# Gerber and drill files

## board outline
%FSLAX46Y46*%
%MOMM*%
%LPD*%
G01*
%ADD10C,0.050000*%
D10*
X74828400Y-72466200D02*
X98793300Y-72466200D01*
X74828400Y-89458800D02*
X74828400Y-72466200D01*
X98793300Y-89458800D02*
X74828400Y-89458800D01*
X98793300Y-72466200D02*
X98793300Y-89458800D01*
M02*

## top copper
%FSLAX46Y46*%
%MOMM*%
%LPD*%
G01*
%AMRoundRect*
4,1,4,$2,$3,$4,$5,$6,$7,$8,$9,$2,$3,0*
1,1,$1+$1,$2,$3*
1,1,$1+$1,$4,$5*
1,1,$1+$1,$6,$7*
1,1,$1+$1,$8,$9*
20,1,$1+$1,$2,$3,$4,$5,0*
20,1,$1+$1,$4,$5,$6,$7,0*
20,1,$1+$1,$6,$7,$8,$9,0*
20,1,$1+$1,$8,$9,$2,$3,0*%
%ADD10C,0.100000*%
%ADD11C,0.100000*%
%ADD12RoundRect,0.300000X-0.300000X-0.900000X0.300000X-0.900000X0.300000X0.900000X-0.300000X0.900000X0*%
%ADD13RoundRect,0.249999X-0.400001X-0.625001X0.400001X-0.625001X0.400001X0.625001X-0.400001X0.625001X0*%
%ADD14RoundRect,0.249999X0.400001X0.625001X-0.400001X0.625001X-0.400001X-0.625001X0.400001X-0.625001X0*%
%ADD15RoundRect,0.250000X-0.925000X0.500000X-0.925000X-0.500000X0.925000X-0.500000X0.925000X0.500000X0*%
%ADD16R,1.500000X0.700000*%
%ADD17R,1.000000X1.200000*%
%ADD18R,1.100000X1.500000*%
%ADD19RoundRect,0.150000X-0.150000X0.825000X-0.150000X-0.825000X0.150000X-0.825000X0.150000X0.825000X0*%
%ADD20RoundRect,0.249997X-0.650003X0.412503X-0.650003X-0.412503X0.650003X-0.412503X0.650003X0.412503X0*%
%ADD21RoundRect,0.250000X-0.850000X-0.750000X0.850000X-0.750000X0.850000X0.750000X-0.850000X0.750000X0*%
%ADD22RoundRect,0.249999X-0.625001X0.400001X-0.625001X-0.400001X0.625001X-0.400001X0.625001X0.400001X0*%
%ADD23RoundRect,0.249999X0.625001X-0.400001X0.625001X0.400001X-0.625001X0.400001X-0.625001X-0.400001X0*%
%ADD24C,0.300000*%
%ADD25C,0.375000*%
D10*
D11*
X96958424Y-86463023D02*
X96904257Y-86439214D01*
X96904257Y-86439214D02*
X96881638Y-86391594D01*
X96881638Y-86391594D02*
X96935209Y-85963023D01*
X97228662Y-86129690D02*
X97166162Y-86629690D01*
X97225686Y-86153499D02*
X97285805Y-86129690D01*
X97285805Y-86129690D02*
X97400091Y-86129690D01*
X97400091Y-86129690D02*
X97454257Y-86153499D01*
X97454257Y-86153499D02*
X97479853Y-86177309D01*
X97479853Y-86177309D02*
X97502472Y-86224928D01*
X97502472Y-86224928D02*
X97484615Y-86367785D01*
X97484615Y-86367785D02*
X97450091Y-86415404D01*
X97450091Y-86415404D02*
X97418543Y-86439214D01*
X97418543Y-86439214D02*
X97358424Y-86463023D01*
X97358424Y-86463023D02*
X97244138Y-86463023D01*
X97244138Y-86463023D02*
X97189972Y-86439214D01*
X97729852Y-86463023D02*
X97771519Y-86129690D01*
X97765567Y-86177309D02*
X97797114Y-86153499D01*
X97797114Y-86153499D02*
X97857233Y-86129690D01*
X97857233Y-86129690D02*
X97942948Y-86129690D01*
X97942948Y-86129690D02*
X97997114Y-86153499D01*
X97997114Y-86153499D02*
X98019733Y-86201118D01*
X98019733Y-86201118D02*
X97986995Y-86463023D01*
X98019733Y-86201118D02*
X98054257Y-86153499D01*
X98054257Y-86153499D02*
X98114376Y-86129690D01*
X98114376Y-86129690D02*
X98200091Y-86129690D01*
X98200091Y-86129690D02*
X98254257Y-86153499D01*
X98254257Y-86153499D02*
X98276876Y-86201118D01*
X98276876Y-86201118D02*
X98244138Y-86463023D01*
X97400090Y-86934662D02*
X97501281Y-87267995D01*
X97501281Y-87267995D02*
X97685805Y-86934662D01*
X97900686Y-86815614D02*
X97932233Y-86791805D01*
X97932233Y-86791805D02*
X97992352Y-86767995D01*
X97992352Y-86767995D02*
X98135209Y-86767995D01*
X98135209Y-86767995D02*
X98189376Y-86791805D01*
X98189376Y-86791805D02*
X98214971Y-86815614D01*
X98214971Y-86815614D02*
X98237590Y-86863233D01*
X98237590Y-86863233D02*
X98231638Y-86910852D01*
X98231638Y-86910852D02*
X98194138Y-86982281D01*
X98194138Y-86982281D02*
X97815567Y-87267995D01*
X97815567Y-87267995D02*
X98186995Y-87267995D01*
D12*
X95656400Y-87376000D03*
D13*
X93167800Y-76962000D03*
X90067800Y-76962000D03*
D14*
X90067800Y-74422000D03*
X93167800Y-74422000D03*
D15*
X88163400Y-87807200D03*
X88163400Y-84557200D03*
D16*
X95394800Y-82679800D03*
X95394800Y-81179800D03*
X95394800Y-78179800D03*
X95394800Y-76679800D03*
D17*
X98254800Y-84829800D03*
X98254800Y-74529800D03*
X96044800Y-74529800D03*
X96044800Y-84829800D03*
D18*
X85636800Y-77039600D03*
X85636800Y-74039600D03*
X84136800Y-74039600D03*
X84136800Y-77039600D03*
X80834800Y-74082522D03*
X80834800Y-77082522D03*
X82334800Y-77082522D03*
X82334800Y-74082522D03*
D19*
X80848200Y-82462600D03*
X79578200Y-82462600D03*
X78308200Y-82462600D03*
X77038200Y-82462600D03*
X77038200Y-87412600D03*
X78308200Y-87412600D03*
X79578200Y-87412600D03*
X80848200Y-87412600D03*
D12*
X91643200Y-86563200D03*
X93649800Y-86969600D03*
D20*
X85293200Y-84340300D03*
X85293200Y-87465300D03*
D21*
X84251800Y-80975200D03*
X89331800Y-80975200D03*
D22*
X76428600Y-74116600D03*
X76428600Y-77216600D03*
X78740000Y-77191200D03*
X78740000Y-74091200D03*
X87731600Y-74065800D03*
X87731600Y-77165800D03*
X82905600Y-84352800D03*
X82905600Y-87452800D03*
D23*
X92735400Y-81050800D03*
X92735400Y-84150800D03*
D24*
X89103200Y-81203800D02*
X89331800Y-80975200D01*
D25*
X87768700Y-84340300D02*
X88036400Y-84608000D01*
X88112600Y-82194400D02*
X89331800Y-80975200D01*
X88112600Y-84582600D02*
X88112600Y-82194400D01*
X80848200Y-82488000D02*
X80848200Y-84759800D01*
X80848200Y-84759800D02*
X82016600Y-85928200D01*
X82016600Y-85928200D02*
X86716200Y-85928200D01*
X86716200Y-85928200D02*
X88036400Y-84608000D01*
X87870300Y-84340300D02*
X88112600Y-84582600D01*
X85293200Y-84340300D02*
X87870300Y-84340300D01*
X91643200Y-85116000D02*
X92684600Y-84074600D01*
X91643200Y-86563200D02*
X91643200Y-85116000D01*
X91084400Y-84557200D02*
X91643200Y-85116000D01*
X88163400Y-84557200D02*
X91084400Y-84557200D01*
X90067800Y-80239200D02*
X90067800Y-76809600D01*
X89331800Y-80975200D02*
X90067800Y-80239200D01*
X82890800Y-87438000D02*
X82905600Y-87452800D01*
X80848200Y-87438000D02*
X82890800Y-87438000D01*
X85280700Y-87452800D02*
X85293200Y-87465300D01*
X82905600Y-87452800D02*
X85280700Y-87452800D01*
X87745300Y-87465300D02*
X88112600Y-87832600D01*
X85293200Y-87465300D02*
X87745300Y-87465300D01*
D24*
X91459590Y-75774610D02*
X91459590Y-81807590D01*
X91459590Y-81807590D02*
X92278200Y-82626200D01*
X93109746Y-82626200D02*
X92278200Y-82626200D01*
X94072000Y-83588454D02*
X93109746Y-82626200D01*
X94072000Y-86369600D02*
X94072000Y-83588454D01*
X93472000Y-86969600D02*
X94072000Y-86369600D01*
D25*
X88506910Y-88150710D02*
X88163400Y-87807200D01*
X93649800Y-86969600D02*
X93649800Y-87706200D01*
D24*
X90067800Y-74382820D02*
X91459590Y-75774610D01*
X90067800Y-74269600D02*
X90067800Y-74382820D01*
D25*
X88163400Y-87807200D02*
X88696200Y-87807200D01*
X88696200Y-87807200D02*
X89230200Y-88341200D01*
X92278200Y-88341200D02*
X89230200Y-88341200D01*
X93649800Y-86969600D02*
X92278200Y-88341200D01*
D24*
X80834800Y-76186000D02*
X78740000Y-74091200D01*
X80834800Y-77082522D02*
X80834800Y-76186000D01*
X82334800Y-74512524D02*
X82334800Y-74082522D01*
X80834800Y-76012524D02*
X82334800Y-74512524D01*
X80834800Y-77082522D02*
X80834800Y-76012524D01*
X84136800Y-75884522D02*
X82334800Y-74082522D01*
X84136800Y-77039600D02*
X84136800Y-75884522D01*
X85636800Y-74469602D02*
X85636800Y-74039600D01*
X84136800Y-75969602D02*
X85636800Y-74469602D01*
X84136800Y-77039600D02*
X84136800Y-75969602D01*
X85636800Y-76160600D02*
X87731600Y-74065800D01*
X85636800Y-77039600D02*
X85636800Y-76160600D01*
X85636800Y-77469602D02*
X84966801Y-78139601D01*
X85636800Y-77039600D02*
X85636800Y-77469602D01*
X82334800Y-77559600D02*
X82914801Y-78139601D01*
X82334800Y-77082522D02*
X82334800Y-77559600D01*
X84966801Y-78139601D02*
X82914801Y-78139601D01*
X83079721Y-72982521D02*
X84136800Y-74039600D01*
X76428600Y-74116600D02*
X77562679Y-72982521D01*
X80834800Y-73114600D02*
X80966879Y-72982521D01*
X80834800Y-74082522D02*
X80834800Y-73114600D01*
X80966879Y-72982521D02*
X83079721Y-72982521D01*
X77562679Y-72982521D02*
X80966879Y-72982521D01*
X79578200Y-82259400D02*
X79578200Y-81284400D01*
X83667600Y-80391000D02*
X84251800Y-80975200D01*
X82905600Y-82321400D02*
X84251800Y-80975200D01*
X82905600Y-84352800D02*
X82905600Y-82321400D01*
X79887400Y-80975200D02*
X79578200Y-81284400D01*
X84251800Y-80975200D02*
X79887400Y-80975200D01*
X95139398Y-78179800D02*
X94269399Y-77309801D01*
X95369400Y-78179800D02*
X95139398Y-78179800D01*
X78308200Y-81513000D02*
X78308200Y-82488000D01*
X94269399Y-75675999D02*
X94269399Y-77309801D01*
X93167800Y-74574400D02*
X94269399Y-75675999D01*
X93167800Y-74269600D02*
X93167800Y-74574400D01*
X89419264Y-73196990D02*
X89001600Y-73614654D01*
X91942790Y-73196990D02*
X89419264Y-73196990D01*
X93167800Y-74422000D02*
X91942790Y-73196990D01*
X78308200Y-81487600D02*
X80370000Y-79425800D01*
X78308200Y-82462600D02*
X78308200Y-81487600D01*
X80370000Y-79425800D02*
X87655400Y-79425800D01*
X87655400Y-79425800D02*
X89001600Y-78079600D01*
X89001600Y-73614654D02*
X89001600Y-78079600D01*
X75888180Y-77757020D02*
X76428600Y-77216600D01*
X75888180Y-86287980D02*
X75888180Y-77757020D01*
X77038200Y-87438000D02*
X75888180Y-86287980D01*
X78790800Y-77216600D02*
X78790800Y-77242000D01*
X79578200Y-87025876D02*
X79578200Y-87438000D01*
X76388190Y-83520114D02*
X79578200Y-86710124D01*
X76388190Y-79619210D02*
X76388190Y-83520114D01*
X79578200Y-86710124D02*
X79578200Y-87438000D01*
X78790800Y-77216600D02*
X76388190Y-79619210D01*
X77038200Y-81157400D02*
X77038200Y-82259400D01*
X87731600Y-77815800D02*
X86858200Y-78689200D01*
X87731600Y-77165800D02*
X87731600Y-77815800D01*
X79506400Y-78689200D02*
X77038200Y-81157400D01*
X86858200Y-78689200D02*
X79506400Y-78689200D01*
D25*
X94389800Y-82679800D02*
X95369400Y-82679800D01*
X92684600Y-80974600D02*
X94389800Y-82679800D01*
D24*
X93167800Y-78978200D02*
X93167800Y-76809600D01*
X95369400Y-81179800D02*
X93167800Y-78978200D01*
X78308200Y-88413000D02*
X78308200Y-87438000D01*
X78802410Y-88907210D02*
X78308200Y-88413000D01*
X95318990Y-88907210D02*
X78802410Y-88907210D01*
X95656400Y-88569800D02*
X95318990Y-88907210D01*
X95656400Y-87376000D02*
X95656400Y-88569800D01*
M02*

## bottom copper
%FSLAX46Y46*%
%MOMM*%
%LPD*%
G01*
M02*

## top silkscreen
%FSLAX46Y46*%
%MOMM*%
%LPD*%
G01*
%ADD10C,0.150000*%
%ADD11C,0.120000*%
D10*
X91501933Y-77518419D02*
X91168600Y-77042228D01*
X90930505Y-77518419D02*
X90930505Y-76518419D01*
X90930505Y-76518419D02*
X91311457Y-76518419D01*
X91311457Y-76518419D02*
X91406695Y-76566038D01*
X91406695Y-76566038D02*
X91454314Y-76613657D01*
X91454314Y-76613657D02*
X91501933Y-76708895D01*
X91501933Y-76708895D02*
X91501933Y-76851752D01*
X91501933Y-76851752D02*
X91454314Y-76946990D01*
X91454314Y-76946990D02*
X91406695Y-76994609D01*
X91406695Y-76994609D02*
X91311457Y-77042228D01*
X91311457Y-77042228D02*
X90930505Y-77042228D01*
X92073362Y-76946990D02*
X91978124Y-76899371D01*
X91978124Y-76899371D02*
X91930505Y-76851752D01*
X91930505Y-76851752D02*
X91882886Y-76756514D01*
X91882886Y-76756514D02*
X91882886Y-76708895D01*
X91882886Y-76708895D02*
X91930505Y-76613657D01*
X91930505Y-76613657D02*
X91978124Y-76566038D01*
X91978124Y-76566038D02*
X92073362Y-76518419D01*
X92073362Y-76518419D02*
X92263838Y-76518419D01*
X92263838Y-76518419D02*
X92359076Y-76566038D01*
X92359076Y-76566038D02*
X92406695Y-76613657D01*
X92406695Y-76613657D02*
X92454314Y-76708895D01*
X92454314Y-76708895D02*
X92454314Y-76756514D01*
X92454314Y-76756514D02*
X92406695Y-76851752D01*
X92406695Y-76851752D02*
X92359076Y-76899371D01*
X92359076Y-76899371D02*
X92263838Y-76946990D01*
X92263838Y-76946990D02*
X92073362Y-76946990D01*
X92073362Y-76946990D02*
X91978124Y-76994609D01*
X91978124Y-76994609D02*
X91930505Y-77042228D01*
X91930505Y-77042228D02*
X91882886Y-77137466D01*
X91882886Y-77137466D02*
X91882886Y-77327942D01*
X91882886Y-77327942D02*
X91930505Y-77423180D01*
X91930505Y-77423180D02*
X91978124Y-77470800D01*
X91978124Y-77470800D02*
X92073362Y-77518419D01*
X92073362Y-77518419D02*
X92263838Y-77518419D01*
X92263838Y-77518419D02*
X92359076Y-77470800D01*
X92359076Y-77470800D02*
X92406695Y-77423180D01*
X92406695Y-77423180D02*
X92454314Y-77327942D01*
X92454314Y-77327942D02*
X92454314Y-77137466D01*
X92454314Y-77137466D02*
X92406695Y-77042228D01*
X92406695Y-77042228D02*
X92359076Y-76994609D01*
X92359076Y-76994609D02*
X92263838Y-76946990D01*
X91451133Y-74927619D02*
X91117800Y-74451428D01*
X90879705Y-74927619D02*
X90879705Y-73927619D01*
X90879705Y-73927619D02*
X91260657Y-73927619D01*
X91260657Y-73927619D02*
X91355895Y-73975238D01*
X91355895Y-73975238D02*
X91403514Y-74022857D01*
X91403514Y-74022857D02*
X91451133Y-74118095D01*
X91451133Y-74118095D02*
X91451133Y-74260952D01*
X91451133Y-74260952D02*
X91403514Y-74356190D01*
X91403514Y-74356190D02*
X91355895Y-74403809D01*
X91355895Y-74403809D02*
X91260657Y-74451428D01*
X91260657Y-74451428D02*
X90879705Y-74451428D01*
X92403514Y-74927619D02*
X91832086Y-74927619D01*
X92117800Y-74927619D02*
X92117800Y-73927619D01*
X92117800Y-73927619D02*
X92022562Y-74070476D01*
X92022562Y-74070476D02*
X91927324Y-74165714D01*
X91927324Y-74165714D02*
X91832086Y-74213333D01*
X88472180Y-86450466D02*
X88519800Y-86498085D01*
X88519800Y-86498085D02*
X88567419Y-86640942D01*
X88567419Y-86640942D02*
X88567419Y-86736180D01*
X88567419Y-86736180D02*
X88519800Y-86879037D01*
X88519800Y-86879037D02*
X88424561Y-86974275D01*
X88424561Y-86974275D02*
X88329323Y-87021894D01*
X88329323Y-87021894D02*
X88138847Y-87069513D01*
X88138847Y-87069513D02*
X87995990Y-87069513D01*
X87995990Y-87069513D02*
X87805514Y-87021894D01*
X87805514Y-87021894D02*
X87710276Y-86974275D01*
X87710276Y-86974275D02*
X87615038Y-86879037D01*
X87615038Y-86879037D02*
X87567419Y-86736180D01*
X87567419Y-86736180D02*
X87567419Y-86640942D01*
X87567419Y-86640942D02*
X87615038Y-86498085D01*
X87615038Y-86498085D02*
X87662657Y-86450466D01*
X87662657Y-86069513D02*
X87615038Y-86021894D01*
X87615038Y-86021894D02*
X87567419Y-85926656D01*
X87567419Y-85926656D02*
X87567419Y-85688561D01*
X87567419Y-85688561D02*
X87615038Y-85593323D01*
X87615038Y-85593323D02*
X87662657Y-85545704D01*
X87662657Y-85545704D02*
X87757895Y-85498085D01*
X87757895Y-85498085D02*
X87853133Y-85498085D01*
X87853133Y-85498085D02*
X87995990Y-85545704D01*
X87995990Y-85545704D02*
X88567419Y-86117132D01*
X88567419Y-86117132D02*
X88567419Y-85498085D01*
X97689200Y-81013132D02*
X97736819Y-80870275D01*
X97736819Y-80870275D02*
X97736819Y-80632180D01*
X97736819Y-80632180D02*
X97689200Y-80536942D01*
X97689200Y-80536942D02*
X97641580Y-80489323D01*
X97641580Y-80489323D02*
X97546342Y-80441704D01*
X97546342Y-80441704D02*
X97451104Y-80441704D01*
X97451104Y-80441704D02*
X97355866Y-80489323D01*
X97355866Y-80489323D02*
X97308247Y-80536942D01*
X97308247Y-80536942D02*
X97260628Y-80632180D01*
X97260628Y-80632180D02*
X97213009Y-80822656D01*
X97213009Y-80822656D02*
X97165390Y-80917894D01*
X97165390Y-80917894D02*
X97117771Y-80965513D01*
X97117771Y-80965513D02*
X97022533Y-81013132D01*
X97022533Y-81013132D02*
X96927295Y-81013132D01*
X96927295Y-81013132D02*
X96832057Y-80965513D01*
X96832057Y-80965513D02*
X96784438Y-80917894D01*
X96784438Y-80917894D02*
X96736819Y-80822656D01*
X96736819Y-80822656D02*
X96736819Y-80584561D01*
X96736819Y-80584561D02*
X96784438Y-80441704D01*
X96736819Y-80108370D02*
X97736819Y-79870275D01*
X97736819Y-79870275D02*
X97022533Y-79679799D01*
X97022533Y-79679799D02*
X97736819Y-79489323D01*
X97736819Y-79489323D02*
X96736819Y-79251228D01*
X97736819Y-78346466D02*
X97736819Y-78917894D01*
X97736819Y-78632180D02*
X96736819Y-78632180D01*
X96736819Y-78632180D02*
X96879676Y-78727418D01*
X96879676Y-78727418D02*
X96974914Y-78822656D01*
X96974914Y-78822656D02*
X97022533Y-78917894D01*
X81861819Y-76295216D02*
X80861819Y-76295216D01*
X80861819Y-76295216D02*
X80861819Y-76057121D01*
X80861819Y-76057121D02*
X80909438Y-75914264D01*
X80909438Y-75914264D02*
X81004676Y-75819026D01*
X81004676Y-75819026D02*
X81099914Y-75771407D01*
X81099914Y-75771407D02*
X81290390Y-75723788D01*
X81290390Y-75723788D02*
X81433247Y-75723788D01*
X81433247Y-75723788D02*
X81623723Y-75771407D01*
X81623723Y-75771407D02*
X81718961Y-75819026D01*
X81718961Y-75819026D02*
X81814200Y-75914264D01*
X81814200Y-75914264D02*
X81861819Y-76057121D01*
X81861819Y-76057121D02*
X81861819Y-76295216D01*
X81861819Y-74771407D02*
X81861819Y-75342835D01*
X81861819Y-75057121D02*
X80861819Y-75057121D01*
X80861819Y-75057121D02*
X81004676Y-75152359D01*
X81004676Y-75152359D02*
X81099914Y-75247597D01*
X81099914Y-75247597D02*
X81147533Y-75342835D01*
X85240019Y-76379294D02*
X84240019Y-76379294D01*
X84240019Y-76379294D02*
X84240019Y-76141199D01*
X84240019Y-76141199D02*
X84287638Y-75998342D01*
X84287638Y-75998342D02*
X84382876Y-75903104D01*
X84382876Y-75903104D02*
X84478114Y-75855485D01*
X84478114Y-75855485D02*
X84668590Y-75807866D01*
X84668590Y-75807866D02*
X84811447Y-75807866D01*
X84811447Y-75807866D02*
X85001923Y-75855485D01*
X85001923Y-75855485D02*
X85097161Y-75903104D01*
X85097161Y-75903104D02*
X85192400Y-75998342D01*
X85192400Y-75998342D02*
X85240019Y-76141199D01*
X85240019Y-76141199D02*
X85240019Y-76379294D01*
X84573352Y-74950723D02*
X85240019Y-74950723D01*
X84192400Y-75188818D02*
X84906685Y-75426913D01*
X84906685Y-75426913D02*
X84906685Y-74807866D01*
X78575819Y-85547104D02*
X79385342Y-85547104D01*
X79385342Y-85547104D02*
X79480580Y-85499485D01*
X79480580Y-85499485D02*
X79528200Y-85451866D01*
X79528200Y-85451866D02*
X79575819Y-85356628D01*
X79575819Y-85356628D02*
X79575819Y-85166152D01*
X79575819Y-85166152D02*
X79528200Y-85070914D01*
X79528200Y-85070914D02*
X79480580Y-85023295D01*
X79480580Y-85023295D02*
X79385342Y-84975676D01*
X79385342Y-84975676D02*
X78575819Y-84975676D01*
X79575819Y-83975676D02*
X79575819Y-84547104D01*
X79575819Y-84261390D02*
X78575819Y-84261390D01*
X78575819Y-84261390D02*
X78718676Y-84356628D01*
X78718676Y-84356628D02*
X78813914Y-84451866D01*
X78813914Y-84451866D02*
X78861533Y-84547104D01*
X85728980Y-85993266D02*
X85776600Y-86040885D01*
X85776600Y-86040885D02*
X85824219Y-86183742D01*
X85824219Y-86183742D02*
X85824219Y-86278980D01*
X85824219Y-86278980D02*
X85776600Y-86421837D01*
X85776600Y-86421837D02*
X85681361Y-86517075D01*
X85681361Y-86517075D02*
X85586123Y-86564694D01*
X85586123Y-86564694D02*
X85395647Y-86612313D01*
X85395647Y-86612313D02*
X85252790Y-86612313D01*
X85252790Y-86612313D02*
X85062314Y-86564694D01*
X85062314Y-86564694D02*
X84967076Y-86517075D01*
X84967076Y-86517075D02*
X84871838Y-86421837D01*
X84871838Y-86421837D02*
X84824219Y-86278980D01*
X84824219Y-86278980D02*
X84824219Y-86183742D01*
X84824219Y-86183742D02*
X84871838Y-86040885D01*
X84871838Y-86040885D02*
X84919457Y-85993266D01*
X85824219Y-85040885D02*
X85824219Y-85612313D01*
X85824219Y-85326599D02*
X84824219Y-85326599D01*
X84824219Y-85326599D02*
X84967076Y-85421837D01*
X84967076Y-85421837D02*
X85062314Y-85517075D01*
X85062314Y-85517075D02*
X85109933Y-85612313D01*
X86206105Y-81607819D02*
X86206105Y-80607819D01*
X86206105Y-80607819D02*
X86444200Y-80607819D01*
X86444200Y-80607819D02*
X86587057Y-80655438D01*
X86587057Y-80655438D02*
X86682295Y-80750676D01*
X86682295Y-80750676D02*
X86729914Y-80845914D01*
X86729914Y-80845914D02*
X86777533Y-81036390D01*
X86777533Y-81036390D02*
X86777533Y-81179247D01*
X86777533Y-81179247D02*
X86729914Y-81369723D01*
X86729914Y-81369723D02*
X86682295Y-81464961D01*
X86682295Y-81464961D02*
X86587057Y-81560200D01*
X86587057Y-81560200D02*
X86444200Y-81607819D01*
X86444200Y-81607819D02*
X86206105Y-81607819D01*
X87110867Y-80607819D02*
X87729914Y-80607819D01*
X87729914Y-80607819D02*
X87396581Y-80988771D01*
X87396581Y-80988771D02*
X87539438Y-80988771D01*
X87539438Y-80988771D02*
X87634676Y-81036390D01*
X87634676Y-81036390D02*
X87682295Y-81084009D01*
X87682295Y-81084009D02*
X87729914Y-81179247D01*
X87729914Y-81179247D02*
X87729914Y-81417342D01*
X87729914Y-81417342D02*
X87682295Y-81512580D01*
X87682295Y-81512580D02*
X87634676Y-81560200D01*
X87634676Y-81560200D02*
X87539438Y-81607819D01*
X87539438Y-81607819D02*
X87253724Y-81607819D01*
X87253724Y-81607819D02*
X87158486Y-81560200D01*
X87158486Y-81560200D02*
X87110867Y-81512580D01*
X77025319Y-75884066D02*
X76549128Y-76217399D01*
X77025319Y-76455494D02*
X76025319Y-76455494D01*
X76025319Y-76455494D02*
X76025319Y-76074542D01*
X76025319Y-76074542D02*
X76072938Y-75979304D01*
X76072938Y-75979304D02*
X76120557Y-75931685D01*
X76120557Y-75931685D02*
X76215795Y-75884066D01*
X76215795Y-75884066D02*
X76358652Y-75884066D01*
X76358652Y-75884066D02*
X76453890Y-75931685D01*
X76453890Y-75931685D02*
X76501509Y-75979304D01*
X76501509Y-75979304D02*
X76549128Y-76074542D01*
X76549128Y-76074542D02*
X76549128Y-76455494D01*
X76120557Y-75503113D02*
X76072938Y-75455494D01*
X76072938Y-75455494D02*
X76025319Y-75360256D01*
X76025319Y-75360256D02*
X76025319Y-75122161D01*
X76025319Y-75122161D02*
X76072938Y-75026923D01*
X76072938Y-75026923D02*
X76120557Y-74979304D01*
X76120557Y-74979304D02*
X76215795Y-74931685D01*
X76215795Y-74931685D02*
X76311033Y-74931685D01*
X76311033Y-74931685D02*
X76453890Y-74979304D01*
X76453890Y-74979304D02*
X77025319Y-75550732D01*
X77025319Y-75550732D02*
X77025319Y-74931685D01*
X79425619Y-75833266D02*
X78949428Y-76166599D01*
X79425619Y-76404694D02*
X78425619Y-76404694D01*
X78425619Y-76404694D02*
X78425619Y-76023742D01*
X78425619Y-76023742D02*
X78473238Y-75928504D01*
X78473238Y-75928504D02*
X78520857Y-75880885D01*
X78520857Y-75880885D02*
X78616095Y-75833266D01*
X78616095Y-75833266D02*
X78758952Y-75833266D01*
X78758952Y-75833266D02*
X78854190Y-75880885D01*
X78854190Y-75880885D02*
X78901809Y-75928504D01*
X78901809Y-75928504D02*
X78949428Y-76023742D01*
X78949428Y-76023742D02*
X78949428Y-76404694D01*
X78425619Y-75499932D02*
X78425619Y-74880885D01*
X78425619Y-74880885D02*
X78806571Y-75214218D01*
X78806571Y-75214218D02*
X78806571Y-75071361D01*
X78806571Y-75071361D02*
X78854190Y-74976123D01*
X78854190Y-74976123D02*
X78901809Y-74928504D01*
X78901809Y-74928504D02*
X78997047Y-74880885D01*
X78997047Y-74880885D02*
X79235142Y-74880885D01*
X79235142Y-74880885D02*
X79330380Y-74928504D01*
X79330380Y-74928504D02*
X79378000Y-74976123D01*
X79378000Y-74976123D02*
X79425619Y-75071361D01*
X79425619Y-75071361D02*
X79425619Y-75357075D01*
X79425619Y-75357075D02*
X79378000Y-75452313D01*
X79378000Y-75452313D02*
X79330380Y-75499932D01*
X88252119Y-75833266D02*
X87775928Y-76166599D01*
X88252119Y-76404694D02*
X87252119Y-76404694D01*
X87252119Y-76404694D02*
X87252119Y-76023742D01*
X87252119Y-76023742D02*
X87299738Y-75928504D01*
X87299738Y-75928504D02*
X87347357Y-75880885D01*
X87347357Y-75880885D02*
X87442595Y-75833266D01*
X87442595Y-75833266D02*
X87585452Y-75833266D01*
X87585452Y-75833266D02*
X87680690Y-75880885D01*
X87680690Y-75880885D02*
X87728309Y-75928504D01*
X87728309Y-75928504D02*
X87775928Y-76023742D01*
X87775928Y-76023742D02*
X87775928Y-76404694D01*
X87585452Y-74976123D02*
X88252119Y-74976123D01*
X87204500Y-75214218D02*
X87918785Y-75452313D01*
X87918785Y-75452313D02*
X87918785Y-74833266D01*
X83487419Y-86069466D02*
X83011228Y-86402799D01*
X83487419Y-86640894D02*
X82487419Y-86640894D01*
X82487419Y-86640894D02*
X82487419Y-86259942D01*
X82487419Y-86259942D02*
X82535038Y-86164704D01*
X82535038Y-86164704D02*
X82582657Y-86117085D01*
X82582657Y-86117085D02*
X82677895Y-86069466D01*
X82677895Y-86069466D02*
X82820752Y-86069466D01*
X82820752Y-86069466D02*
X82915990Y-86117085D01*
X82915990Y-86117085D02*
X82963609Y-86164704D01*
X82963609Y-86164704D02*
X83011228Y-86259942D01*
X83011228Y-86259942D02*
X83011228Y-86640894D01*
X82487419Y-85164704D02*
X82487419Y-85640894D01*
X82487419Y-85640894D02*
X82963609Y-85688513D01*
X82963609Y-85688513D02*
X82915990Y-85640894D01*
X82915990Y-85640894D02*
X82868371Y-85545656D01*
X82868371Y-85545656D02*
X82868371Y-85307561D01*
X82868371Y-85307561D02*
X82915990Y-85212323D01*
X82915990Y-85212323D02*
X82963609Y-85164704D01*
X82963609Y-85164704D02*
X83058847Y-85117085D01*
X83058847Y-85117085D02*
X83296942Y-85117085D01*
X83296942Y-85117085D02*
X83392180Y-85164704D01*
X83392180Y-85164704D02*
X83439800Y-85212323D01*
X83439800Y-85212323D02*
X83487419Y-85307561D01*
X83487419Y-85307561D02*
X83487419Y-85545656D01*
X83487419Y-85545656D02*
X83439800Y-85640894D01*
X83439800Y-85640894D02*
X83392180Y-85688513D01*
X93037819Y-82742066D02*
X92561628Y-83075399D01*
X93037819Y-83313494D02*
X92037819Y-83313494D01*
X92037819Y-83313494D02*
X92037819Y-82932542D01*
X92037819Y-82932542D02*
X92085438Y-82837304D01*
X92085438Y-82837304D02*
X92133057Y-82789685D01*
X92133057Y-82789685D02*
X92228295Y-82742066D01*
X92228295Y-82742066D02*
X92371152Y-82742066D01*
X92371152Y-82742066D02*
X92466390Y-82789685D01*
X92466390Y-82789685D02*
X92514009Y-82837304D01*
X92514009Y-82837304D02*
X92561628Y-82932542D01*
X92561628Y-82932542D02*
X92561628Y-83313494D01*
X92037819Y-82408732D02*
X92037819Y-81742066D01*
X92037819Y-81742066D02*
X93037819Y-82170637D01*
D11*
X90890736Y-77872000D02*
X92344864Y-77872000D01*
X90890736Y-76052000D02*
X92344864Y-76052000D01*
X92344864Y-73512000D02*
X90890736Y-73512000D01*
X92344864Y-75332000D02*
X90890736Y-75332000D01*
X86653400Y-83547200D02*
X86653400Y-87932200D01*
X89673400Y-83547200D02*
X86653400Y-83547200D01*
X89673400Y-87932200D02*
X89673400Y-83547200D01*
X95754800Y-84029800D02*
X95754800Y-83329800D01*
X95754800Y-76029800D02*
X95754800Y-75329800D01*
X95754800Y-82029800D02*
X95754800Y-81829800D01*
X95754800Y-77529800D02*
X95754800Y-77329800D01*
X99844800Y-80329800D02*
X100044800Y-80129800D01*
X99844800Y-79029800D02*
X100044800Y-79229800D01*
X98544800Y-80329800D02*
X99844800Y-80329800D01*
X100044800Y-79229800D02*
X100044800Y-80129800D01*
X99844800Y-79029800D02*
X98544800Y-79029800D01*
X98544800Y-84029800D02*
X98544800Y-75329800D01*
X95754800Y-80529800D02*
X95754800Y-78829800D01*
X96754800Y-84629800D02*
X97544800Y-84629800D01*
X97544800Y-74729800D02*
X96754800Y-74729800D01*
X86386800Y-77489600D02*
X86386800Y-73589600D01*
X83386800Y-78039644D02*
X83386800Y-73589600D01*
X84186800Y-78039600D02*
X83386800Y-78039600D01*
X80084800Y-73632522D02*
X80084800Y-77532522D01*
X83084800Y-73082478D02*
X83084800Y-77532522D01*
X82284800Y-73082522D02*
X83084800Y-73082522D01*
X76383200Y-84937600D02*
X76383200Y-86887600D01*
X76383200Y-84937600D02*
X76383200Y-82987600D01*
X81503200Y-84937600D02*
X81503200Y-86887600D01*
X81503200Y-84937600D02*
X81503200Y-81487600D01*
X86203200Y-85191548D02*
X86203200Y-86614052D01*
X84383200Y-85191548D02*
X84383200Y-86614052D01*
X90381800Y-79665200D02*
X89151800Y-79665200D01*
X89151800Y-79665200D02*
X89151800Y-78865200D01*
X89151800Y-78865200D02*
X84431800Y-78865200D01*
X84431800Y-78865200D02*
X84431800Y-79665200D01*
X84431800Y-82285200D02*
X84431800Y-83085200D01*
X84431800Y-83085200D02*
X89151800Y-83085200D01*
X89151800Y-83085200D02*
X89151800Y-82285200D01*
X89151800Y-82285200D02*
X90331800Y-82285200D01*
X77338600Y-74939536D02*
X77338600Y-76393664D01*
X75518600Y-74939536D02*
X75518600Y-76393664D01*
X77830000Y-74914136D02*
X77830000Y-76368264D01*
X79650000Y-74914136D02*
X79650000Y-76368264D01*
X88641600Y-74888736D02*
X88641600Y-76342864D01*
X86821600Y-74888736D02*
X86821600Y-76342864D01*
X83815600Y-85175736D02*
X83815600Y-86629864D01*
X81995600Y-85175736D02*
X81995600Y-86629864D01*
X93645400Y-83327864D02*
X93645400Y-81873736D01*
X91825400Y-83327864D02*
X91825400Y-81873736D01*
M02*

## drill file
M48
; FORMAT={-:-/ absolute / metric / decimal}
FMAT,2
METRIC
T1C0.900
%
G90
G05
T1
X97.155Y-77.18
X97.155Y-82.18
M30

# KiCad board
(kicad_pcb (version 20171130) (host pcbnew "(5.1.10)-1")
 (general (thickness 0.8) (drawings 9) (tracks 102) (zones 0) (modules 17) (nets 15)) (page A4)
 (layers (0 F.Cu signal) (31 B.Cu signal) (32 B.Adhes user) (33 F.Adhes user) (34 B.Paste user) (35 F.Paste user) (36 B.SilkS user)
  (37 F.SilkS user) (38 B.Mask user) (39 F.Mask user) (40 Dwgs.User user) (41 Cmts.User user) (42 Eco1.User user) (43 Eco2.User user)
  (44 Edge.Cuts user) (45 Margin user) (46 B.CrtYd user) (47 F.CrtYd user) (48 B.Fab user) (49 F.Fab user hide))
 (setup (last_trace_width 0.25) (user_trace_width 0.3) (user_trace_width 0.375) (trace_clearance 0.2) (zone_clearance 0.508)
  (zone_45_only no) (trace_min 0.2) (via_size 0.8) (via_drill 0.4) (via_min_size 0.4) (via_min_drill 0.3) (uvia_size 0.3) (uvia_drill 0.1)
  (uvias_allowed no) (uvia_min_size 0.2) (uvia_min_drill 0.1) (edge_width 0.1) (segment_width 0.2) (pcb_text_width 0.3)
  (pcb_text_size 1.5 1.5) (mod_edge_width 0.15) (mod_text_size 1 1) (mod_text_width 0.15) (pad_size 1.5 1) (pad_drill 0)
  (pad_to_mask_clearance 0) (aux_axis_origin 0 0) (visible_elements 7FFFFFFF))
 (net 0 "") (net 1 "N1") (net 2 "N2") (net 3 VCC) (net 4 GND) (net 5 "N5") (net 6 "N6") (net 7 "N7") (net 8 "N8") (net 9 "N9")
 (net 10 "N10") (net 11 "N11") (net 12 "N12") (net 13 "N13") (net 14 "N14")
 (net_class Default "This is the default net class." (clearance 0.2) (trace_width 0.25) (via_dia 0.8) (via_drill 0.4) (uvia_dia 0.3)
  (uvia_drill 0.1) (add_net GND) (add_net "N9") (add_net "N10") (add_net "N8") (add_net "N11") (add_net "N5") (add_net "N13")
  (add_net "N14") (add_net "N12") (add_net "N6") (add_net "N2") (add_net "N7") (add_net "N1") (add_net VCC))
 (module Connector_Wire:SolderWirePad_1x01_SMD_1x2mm (layer F.Cu) (at 95.6564 87.376)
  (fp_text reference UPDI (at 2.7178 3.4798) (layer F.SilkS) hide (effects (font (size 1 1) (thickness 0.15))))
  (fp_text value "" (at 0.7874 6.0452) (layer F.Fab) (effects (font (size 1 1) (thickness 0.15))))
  (pad 1 smd roundrect (at 0 0) (size 1.2 2.4) (layers F.Cu F.Mask) (roundrect_rratio 0.25) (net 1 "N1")))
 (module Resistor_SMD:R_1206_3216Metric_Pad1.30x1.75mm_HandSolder (layer F.Cu) (at 91.6178 76.962)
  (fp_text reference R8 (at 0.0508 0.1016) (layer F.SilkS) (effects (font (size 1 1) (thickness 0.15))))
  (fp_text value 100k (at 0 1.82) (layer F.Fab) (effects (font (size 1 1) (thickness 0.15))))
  (fp_line (start -0.727064 0.91) (end 0.727064 0.91) (layer F.SilkS) (width 0.12))
  (fp_line (start -0.727064 -0.91) (end 0.727064 -0.91) (layer F.SilkS) (width 0.12))
  (pad 2 smd roundrect (at 1.55 0) (size 1.3 1.75) (layers F.Cu F.Paste F.Mask) (roundrect_rratio 0.1923069230769231) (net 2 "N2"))
  (pad 1 smd roundrect (at -1.55 0) (size 1.3 1.75) (layers F.Cu F.Paste F.Mask) (roundrect_rratio 0.1923069230769231) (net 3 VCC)))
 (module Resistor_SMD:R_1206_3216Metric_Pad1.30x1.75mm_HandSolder (layer F.Cu) (at 91.6178 74.422 180)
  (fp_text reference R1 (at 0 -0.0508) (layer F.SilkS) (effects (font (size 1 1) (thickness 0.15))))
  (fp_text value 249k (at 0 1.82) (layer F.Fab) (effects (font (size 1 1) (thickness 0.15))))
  (fp_line (start -0.727064 0.91) (end 0.727064 0.91) (layer F.SilkS) (width 0.12))
  (fp_line (start -0.727064 -0.91) (end 0.727064 -0.91) (layer F.SilkS) (width 0.12))
  (pad 2 smd roundrect (at 1.55 0 180) (size 1.3 1.75) (layers F.Cu F.Paste F.Mask) (roundrect_rratio 0.1923069230769231) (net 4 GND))
  (pad 1 smd roundrect (at -1.55 0 180) (size 1.3 1.75) (layers F.Cu F.Paste F.Mask) (roundrect_rratio 0.1923069230769231) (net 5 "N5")))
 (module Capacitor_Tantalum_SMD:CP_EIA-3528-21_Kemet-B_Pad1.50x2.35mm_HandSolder (layer F.Cu) (at 88.1634 86.1822 270)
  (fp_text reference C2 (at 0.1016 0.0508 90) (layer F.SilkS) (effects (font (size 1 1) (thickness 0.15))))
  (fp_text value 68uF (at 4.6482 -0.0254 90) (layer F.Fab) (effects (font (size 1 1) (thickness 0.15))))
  (fp_line (start -2.635 1.51) (end 1.75 1.51) (layer F.SilkS) (width 0.12))
  (fp_line (start -2.635 -1.51) (end -2.635 1.51) (layer F.SilkS) (width 0.12))
  (fp_line (start 1.75 -1.51) (end -2.635 -1.51) (layer F.SilkS) (width 0.12))
  (pad 2 smd roundrect (at 1.625 0 270) (size 1.5 2.35) (layers F.Cu F.Paste F.Mask) (roundrect_rratio 0.1666666666666667) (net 4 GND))
  (pad 1 smd roundrect (at -1.625 0 270) (size 1.5 2.35) (layers F.Cu F.Paste F.Mask) (roundrect_rratio 0.1666666666666667) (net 3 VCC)))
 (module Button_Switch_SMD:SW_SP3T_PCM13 (layer F.Cu) (at 96.8248 79.6798 90)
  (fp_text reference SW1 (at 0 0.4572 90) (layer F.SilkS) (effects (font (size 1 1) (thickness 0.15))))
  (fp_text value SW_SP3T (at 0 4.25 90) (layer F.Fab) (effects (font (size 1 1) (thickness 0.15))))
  (fp_line (start -4.35 -1.07) (end -3.65 -1.07) (layer F.SilkS) (width 0.12))
  (fp_line (start 3.65 -1.07) (end 4.35 -1.07) (layer F.SilkS) (width 0.12))
  (fp_line (start -2.35 -1.07) (end -2.15 -1.07) (layer F.SilkS) (width 0.12))
  (fp_line (start 2.15 -1.07) (end 2.35 -1.07) (layer F.SilkS) (width 0.12))
  (fp_line (start -0.65 3.02) (end -0.45 3.22) (layer F.SilkS) (width 0.12))
  (fp_line (start 0.65 3.02) (end 0.45 3.22) (layer F.SilkS) (width 0.12))
  (fp_line (start -0.65 1.72) (end -0.65 3.02) (layer F.SilkS) (width 0.12))
  (fp_line (start 0.45 3.22) (end -0.45 3.22) (layer F.SilkS) (width 0.12))
  (fp_line (start 0.65 3.02) (end 0.65 1.72) (layer F.SilkS) (width 0.12))
  (fp_line (start -4.35 1.72) (end 4.35 1.72) (layer F.SilkS) (width 0.12))
  (fp_line (start -0.85 -1.07) (end 0.85 -1.07) (layer F.SilkS) (width 0.12))
  (fp_line (start -4.95 -0.07) (end -4.95 0.72) (layer F.SilkS) (width 0.12))
  (fp_line (start 4.95 0.72) (end 4.95 -0.07) (layer F.SilkS) (width 0.12))
  (pad "" np_thru_hole circle (at -2.5 0.33 90) (size 0.9 0.9) (drill 0.9) (layers *.Cu *.Mask))
  (pad "" np_thru_hole circle (at 2.5 0.33 90) (size 0.9 0.9) (drill 0.9) (layers *.Cu *.Mask))
  (pad 1 smd rect (at -3 -1.43 90) (size 0.7 1.5) (layers F.Cu F.Paste F.Mask) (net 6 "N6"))
  (pad 2 smd rect (at -1.5 -1.43 90) (size 0.7 1.5) (layers F.Cu F.Paste F.Mask) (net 2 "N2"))
  (pad 3 smd rect (at 1.5 -1.43 90) (size 0.7 1.5) (layers F.Cu F.Paste F.Mask) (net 5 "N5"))
  (pad 4 smd rect (at 3 -1.43 90) (size 0.7 1.5) (layers F.Cu F.Paste F.Mask) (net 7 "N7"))
  (pad "" smd rect (at -5.15 1.43 90) (size 1.2 1) (layers F.Cu F.Paste F.Mask))
  (pad "" smd rect (at 5.15 1.43 90) (size 1.2 1) (layers F.Cu F.Paste F.Mask))
  (pad "" smd rect (at 5.15 -0.78 90) (size 1.2 1) (layers F.Cu F.Paste F.Mask))
  (pad "" smd rect (at -5.15 -0.78 90) (size 1.2 1) (layers F.Cu F.Paste F.Mask)))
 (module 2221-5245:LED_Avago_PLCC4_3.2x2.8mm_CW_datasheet (layer F.Cu) (at 84.8868 75.5396 90)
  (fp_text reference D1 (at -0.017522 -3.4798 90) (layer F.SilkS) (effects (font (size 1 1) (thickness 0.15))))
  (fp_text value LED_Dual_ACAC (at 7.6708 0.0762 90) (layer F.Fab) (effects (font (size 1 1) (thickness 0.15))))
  (fp_line (start -1.95 1.5) (end 1.95 1.5) (layer F.SilkS) (width 0.12))
  (fp_line (start -2.500044 -1.5) (end 1.95 -1.5) (layer F.SilkS) (width 0.12))
  (fp_line (start -2.5 -0.7) (end -2.5 -1.5) (layer F.SilkS) (width 0.12))
  (pad 3 smd rect (at -1.5 0.75 90) (size 1.5 1.1) (layers F.Cu F.Paste F.Mask) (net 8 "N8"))
  (pad 4 smd rect (at 1.5 0.75 90) (size 1.5 1.1) (layers F.Cu F.Paste F.Mask) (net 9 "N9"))
  (pad 2 smd rect (at 1.5 -0.75 90) (size 1.5 1.1) (layers F.Cu F.Paste F.Mask) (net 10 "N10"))
  (pad 1 smd rect (at -1.5 -0.75 90) (size 1.5 1.1) (layers F.Cu F.Paste F.Mask) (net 9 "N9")))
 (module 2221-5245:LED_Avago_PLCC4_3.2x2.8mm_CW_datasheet (layer F.Cu) (at 81.5848 75.582522 270)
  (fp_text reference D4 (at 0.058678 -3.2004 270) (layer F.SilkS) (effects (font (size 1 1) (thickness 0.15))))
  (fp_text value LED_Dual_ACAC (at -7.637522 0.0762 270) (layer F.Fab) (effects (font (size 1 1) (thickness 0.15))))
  (fp_line (start -1.95 1.5) (end 1.95 1.5) (layer F.SilkS) (width 0.12))
  (fp_line (start -2.500044 -1.5) (end 1.95 -1.5) (layer F.SilkS) (width 0.12))
  (fp_line (start -2.5 -0.7) (end -2.5 -1.5) (layer F.SilkS) (width 0.12))
  (pad 3 smd rect (at -1.5 0.75 270) (size 1.5 1.1) (layers F.Cu F.Paste F.Mask) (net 10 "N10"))
  (pad 4 smd rect (at 1.5 0.75 270) (size 1.5 1.1) (layers F.Cu F.Paste F.Mask) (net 9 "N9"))
  (pad 2 smd rect (at 1.5 -0.75 270) (size 1.5 1.1) (layers F.Cu F.Paste F.Mask) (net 8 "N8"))
  (pad 1 smd rect (at -1.5 -0.75 270) (size 1.5 1.1) (layers F.Cu F.Paste F.Mask) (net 9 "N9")))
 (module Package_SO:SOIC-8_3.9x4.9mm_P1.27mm (layer F.Cu) (at 78.9432 84.9376 270)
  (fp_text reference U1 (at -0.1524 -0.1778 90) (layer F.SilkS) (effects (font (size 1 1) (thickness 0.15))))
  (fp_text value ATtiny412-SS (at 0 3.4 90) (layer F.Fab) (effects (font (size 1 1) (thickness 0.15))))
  (fp_line (start 0 2.56) (end 1.95 2.56) (layer F.SilkS) (width 0.12))
  (fp_line (start 0 2.56) (end -1.95 2.56) (layer F.SilkS) (width 0.12))
  (fp_line (start 0 -2.56) (end 1.95 -2.56) (layer F.SilkS) (width 0.12))
  (fp_line (start 0 -2.56) (end -3.45 -2.56) (layer F.SilkS) (width 0.12))
  (pad 1 smd roundrect (at -2.475 -1.905 270) (size 1.95 0.6) (layers F.Cu F.Paste F.Mask) (roundrect_rratio 0.25) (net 3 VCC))
  (pad 2 smd roundrect (at -2.475 -0.635 270) (size 1.95 0.6) (layers F.Cu F.Paste F.Mask) (roundrect_rratio 0.25) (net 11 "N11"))
  (pad 3 smd roundrect (at -2.475 0.635 270) (size 1.95 0.6) (layers F.Cu F.Paste F.Mask) (roundrect_rratio 0.25) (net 5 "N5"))
  (pad 4 smd roundrect (at -2.475 1.905 270) (size 1.95 0.6) (layers F.Cu F.Paste F.Mask) (roundrect_rratio 0.25) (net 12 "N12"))
  (pad 5 smd roundrect (at 2.475 1.905 270) (size 1.95 0.6) (layers F.Cu F.Paste F.Mask) (roundrect_rratio 0.25) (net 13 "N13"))
  (pad 6 smd roundrect (at 2.475 0.635 270) (size 1.95 0.6) (layers F.Cu F.Paste F.Mask) (roundrect_rratio 0.25) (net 1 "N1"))
  (pad 7 smd roundrect (at 2.475 -0.635 270) (size 1.95 0.6) (layers F.Cu F.Paste F.Mask) (roundrect_rratio 0.25) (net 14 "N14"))
  (pad 8 smd roundrect (at 2.475 -1.905 270) (size 1.95 0.6) (layers F.Cu F.Paste F.Mask) (roundrect_rratio 0.25) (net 4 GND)))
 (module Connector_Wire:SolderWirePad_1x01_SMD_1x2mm (layer F.Cu) (at 91.6432 86.5632)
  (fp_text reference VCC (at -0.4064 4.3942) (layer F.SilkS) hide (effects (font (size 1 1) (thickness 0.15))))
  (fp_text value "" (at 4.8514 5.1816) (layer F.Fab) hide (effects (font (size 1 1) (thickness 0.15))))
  (pad 1 smd roundrect (at 0 0) (size 1.2 2.4) (layers F.Cu F.Mask) (roundrect_rratio 0.25) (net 3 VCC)))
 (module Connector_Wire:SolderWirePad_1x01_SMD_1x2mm (layer F.Cu) (at 93.6498 86.9696)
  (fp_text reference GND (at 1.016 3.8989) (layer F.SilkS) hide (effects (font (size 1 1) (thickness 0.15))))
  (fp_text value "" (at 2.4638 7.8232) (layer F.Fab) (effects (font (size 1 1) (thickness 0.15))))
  (pad 1 smd roundrect (at 0 0) (size 1.2 2.4) (layers F.Cu F.Mask) (roundrect_rratio 0.25) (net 4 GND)))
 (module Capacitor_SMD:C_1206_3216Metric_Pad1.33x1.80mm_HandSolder (layer F.Cu) (at 85.2932 85.9028 270)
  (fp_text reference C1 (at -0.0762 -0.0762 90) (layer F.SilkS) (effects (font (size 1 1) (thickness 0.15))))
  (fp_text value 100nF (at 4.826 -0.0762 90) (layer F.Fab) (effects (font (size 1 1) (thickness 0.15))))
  (fp_line (start -0.711252 -0.91) (end 0.711252 -0.91) (layer F.SilkS) (width 0.12))
  (fp_line (start -0.711252 0.91) (end 0.711252 0.91) (layer F.SilkS) (width 0.12))
  (pad 1 smd roundrect (at -1.5625 0 270) (size 1.325 1.8) (layers F.Cu F.Paste F.Mask) (roundrect_rratio 0.1886769811320755) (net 3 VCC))
  (pad 2 smd roundrect (at 1.5625 0 270) (size 1.325 1.8) (layers F.Cu F.Paste F.Mask) (roundrect_rratio 0.1886769811320755) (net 4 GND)))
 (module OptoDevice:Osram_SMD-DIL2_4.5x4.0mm (layer F.Cu) (at 86.7918 80.9752 180)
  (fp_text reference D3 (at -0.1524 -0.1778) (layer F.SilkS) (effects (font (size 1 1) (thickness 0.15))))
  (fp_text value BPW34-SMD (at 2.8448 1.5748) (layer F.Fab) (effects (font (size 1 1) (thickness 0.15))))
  (fp_line (start -3.59 1.31) (end -2.36 1.31) (layer F.SilkS) (width 0.12))
  (fp_line (start -2.36 1.31) (end -2.36 2.11) (layer F.SilkS) (width 0.12))
  (fp_line (start -2.36 2.11) (end 2.36 2.11) (layer F.SilkS) (width 0.12))
  (fp_line (start 2.36 2.11) (end 2.36 1.31) (layer F.SilkS) (width 0.12))
  (fp_line (start 2.36 -1.31) (end 2.36 -2.11) (layer F.SilkS) (width 0.12))
  (fp_line (start 2.36 -2.11) (end -2.36 -2.11) (layer F.SilkS) (width 0.12))
  (fp_line (start -2.36 -2.11) (end -2.36 -1.31) (layer F.SilkS) (width 0.12))
  (fp_line (start -2.36 -1.31) (end -3.54 -1.31) (layer F.SilkS) (width 0.12))
  (pad 2 smd roundrect (at 2.54 0) (size 2.2 2) (layers F.Cu F.Paste F.Mask) (roundrect_rratio 0.125) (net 11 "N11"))
  (pad 1 smd roundrect (at -2.54 0) (size 2.2 2) (layers F.Cu F.Paste F.Mask) (roundrect_rratio 0.125) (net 3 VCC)))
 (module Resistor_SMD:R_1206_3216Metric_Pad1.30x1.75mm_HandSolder (layer F.Cu) (at 76.4286 75.6666 270)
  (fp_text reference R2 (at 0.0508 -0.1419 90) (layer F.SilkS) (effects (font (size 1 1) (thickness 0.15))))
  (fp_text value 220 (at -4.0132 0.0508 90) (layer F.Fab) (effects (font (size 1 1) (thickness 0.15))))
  (fp_line (start -0.727064 -0.91) (end 0.727064 -0.91) (layer F.SilkS) (width 0.12))
  (fp_line (start -0.727064 0.91) (end 0.727064 0.91) (layer F.SilkS) (width 0.12))
  (pad 1 smd roundrect (at -1.55 0 270) (size 1.3 1.75) (layers F.Cu F.Paste F.Mask) (roundrect_rratio 0.1923069230769231) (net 10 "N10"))
  (pad 2 smd roundrect (at 1.55 0 270) (size 1.3 1.75) (layers F.Cu F.Paste F.Mask) (roundrect_rratio 0.1923069230769231) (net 13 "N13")))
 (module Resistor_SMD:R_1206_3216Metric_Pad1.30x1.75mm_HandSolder (layer F.Cu) (at 78.74 75.6412 270)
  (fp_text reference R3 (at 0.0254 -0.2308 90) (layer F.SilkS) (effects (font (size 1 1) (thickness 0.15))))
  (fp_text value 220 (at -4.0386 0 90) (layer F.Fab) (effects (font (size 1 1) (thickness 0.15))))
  (fp_line (start -0.727064 0.91) (end 0.727064 0.91) (layer F.SilkS) (width 0.12))
  (fp_line (start -0.727064 -0.91) (end 0.727064 -0.91) (layer F.SilkS) (width 0.12))
  (pad 2 smd roundrect (at 1.55 0 270) (size 1.3 1.75) (layers F.Cu F.Paste F.Mask) (roundrect_rratio 0.1923069230769231) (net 14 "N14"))
  (pad 1 smd roundrect (at -1.55 0 270) (size 1.3 1.75) (layers F.Cu F.Paste F.Mask) (roundrect_rratio 0.1923069230769231) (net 9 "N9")))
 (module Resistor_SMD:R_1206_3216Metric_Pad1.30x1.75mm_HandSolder (layer F.Cu) (at 87.7316 75.6158 270)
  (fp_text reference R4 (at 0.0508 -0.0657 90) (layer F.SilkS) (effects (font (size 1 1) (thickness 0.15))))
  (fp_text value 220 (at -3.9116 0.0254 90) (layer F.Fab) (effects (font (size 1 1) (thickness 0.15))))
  (fp_line (start -0.727064 -0.91) (end 0.727064 -0.91) (layer F.SilkS) (width 0.12))
  (fp_line (start -0.727064 0.91) (end 0.727064 0.91) (layer F.SilkS) (width 0.12))
  (pad 1 smd roundrect (at -1.55 0 270) (size 1.3 1.75) (layers F.Cu F.Paste F.Mask) (roundrect_rratio 0.1923069230769231) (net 8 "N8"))
  (pad 2 smd roundrect (at 1.55 0 270) (size 1.3 1.75) (layers F.Cu F.Paste F.Mask) (roundrect_rratio 0.1923069230769231) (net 12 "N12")))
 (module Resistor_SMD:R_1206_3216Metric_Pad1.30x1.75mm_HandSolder (layer F.Cu) (at 82.9056 85.9028 270)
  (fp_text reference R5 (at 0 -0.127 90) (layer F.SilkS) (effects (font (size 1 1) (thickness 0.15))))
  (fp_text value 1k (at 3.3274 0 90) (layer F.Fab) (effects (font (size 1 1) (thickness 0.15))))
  (fp_line (start -0.727064 -0.91) (end 0.727064 -0.91) (layer F.SilkS) (width 0.12))
  (fp_line (start -0.727064 0.91) (end 0.727064 0.91) (layer F.SilkS) (width 0.12))
  (pad 1 smd roundrect (at -1.55 0 270) (size 1.3 1.75) (layers F.Cu F.Paste F.Mask) (roundrect_rratio 0.1923069230769231) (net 11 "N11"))
  (pad 2 smd roundrect (at 1.55 0 270) (size 1.3 1.75) (layers F.Cu F.Paste F.Mask) (roundrect_rratio 0.1923069230769231) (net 4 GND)))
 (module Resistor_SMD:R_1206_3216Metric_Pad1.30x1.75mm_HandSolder (layer F.Cu) (at 92.7354 82.6008 90)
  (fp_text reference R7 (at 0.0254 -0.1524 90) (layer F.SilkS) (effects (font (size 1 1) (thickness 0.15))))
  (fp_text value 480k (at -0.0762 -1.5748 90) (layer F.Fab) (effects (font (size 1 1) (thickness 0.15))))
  (fp_line (start -0.727064 0.91) (end 0.727064 0.91) (layer F.SilkS) (width 0.12))
  (fp_line (start -0.727064 -0.91) (end 0.727064 -0.91) (layer F.SilkS) (width 0.12))
  (pad 2 smd roundrect (at 1.55 0 90) (size 1.3 1.75) (layers F.Cu F.Paste F.Mask) (roundrect_rratio 0.1923069230769231) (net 6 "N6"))
  (pad 1 smd roundrect (at -1.55 0 90) (size 1.3 1.75) (layers F.Cu F.Paste F.Mask) (roundrect_rratio 0.1923069230769231) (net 3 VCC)))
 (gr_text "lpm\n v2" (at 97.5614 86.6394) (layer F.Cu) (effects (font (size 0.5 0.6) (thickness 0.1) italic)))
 (gr_line (start 74.8284 72.4662) (end 98.7933 72.4662) (layer Edge.Cuts) (width 0.05))
 (gr_line (start 74.8284 89.4588) (end 74.8284 72.4662) (layer Edge.Cuts) (width 0.05))
 (gr_line (start 98.7933 89.4588) (end 74.8284 89.4588) (layer Edge.Cuts) (width 0.05))
 (gr_line (start 98.7933 72.4662) (end 98.7933 89.4588) (layer Edge.Cuts) (width 0.05))
 (segment (start 89.1032 81.2038) (end 89.3318 80.9752) (width 0.3) (layer F.Cu) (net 3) (status 30))
 (segment (start 87.7687 84.3403) (end 88.0364 84.608) (width 0.375) (layer F.Cu) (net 3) (status 30))
 (segment (start 88.1126 82.1944) (end 89.3318 80.9752) (width 0.375) (layer F.Cu) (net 3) (status 20))
 (segment (start 88.1126 84.5826) (end 88.1126 82.1944) (width 0.375) (layer F.Cu) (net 3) (status 10))
 (segment (start 80.8482 82.488) (end 80.8482 84.7598) (width 0.375) (layer F.Cu) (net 3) (status 10))
 (segment (start 80.8482 84.7598) (end 82.0166 85.9282) (width 0.375) (layer F.Cu) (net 3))
 (segment (start 82.0166 85.9282) (end 86.7162 85.9282) (width 0.375) (layer F.Cu) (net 3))
 (segment (start 86.7162 85.9282) (end 88.0364 84.608) (width 0.375) (layer F.Cu) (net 3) (status 20))
 (segment (start 87.8703 84.3403) (end 88.1126 84.5826) (width 0.375) (layer F.Cu) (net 3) (status 30))
 (segment (start 85.2932 84.3403) (end 87.8703 84.3403) (width 0.375) (layer F.Cu) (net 3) (status 30))
 (segment (start 91.6432 85.116) (end 92.6846 84.0746) (width 0.375) (layer F.Cu) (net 3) (status 20))
 (segment (start 91.6432 86.5632) (end 91.6432 85.116) (width 0.375) (layer F.Cu) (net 3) (status 10))
 (segment (start 91.0844 84.5572) (end 91.6432 85.116) (width 0.375) (layer F.Cu) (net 3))
 (segment (start 88.1634 84.5572) (end 91.0844 84.5572) (width 0.375) (layer F.Cu) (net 3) (status 10))
 (segment (start 90.0678 80.2392) (end 90.0678 76.8096) (width 0.375) (layer F.Cu) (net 3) (status 30))
 (segment (start 89.3318 80.9752) (end 90.0678 80.2392) (width 0.375) (layer F.Cu) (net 3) (status 30))
 (segment (start 82.8908 87.438) (end 82.9056 87.4528) (width 0.375) (layer F.Cu) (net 4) (status 30))
 (segment (start 80.8482 87.438) (end 82.8908 87.438) (width 0.375) (layer F.Cu) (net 4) (status 30))
 (segment (start 85.2807 87.4528) (end 85.2932 87.4653) (width 0.375) (layer F.Cu) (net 4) (status 30))
 (segment (start 82.9056 87.4528) (end 85.2807 87.4528) (width 0.375) (layer F.Cu) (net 4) (status 30))
 (segment (start 87.7453 87.4653) (end 88.1126 87.8326) (width 0.375) (layer F.Cu) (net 4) (status 30))
 (segment (start 85.2932 87.4653) (end 87.7453 87.4653) (width 0.375) (layer F.Cu) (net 4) (status 30))
 (segment (start 91.45959 75.77461) (end 91.45959 81.80759) (width 0.3) (layer F.Cu) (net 4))
 (segment (start 91.45959 81.80759) (end 92.2782 82.6262) (width 0.3) (layer F.Cu) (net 4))
 (segment (start 93.109746 82.6262) (end 92.2782 82.6262) (width 0.3) (layer F.Cu) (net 4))
 (segment (start 94.072 83.588454) (end 93.109746 82.6262) (width 0.3) (layer F.Cu) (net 4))
 (segment (start 94.072 86.3696) (end 94.072 83.588454) (width 0.3) (layer F.Cu) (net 4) (status 10))
 (segment (start 93.472 86.9696) (end 94.072 86.3696) (width 0.3) (layer F.Cu) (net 4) (status 30))
 (segment (start 88.50691 88.15071) (end 88.1634 87.8072) (width 0.375) (layer F.Cu) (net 4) (status 30))
 (segment (start 93.6498 86.9696) (end 93.6498 87.7062) (width 0.375) (layer F.Cu) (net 4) (status 30))
 (segment (start 90.0678 74.38282) (end 91.45959 75.77461) (width 0.3) (layer F.Cu) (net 4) (status 10))
 (segment (start 90.0678 74.2696) (end 90.0678 74.38282) (width 0.3) (layer F.Cu) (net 4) (status 30))
 (segment (start 88.1634 87.8072) (end 88.6962 87.8072) (width 0.375) (layer F.Cu) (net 4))
 (segment (start 88.6962 87.8072) (end 89.2302 88.3412) (width 0.375) (layer F.Cu) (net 4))
 (segment (start 92.2782 88.3412) (end 89.2302 88.3412) (width 0.375) (layer F.Cu) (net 4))
 (segment (start 93.6498 86.9696) (end 92.2782 88.3412) (width 0.375) (layer F.Cu) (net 4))
 (segment (start 80.8348 76.186) (end 78.74 74.0912) (width 0.3) (layer F.Cu) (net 9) (status 20))
 (segment (start 80.8348 77.082522) (end 80.8348 76.186) (width 0.3) (layer F.Cu) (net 9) (status 10))
 (segment (start 82.3348 74.512524) (end 82.3348 74.082522) (width 0.3) (layer F.Cu) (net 9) (status 30))
 (segment (start 80.8348 76.012524) (end 82.3348 74.512524) (width 0.3) (layer F.Cu) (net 9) (status 20))
 (segment (start 80.8348 77.082522) (end 80.8348 76.012524) (width 0.3) (layer F.Cu) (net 9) (status 10))
 (segment (start 84.1368 75.884522) (end 82.3348 74.082522) (width 0.3) (layer F.Cu) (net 9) (status 20))
 (segment (start 84.1368 77.0396) (end 84.1368 75.884522) (width 0.3) (layer F.Cu) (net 9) (status 10))
 (segment (start 85.6368 74.469602) (end 85.6368 74.0396) (width 0.3) (layer F.Cu) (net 9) (status 30))
 (segment (start 84.1368 75.969602) (end 85.6368 74.469602) (width 0.3) (layer F.Cu) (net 9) (status 20))
 (segment (start 84.1368 77.0396) (end 84.1368 75.969602) (width 0.3) (layer F.Cu) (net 9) (status 10))
 (segment (start 85.6368 76.1606) (end 87.7316 74.0658) (width 0.3) (layer F.Cu) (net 8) (status 20))
 (segment (start 85.6368 77.0396) (end 85.6368 76.1606) (width 0.3) (layer F.Cu) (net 8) (status 10))
 (segment (start 85.6368 77.469602) (end 84.966801 78.139601) (width 0.3) (layer F.Cu) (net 8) (status 10))
 (segment (start 85.6368 77.0396) (end 85.6368 77.469602) (width 0.3) (layer F.Cu) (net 8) (status 30))
 (segment (start 82.3348 77.5596) (end 82.914801 78.139601) (width 0.3) (layer F.Cu) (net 8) (status 10))
 (segment (start 82.3348 77.082522) (end 82.3348 77.5596) (width 0.3) (layer F.Cu) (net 8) (status 30))
 (segment (start 84.966801 78.139601) (end 82.914801 78.139601) (width 0.3) (layer F.Cu) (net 8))
 (segment (start 83.079721 72.982521) (end 84.1368 74.0396) (width 0.3) (layer F.Cu) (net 10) (status 20))
 (segment (start 76.4286 74.1166) (end 77.562679 72.982521) (width 0.3) (layer F.Cu) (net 10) (status 10))
 (segment (start 80.8348 73.1146) (end 80.966879 72.982521) (width 0.3) (layer F.Cu) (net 10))
 (segment (start 80.8348 74.082522) (end 80.8348 73.1146) (width 0.3) (layer F.Cu) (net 10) (status 10))
 (segment (start 80.966879 72.982521) (end 83.079721 72.982521) (width 0.3) (layer F.Cu) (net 10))
 (segment (start 77.562679 72.982521) (end 80.966879 72.982521) (width 0.3) (layer F.Cu) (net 10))
 (segment (start 79.5782 82.2594) (end 79.5782 81.2844) (width 0.3) (layer F.Cu) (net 11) (status 10))
 (segment (start 83.6676 80.391) (end 84.2518 80.9752) (width 0.3) (layer F.Cu) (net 11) (status 30))
 (segment (start 82.9056 82.3214) (end 84.2518 80.9752) (width 0.3) (layer F.Cu) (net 11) (status 20))
 (segment (start 82.9056 84.3528) (end 82.9056 82.3214) (width 0.3) (layer F.Cu) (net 11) (status 10))
 (segment (start 79.8874 80.9752) (end 79.5782 81.2844) (width 0.3) (layer F.Cu) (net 11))
 (segment (start 84.2518 80.9752) (end 79.8874 80.9752) (width 0.3) (layer F.Cu) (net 11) (status 10))
 (segment (start 95.139398 78.1798) (end 94.269399 77.309801) (width 0.3) (layer F.Cu) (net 5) (status 10))
 (segment (start 95.3694 78.1798) (end 95.139398 78.1798) (width 0.3) (layer F.Cu) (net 5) (status 30))
 (segment (start 78.3082 81.513) (end 78.3082 82.488) (width 0.3) (layer F.Cu) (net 5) (status 30))
 (segment (start 94.269399 75.675999) (end 94.269399 77.309801) (width 0.3) (layer F.Cu) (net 5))
 (segment (start 93.1678 74.5744) (end 94.269399 75.675999) (width 0.3) (layer F.Cu) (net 5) (status 10))
 (segment (start 93.1678 74.2696) (end 93.1678 74.5744) (width 0.3) (layer F.Cu) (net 5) (status 30))
 (segment (start 89.419264 73.19699) (end 89.0016 73.614654) (width 0.3) (layer F.Cu) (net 5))
 (segment (start 91.94279 73.19699) (end 89.419264 73.19699) (width 0.3) (layer F.Cu) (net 5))
 (segment (start 93.1678 74.422) (end 91.94279 73.19699) (width 0.3) (layer F.Cu) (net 5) (status 10))
 (segment (start 78.3082 81.4876) (end 80.37 79.4258) (width 0.3) (layer F.Cu) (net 5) (status 10))
 (segment (start 78.3082 82.4626) (end 78.3082 81.4876) (width 0.3) (layer F.Cu) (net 5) (status 30))
 (segment (start 80.37 79.4258) (end 87.6554 79.4258) (width 0.3) (layer F.Cu) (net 5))
 (segment (start 87.6554 79.4258) (end 89.0016 78.0796) (width 0.3) (layer F.Cu) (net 5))
 (segment (start 89.0016 73.614654) (end 89.0016 78.0796) (width 0.3) (layer F.Cu) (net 5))
 (segment (start 75.88818 77.75702) (end 76.4286 77.2166) (width 0.3) (layer F.Cu) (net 13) (status 30))
 (segment (start 75.88818 86.28798) (end 75.88818 77.75702) (width 0.3) (layer F.Cu) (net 13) (status 20))
 (segment (start 77.0382 87.438) (end 75.88818 86.28798) (width 0.3) (layer F.Cu) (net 13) (status 10))
 (segment (start 78.7908 77.2166) (end 78.7908 77.242) (width 0.3) (layer F.Cu) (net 14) (status 30))
 (segment (start 79.5782 87.025876) (end 79.5782 87.438) (width 0.3) (layer F.Cu) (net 14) (status 30))
 (segment (start 76.38819 83.520114) (end 79.5782 86.710124) (width 0.3) (layer F.Cu) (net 14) (status 20))
 (segment (start 76.38819 79.61921) (end 76.38819 83.520114) (width 0.3) (layer F.Cu) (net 14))
 (segment (start 79.5782 86.710124) (end 79.5782 87.438) (width 0.3) (layer F.Cu) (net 14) (status 30))
 (segment (start 78.7908 77.2166) (end 76.38819 79.61921) (width 0.3) (layer F.Cu) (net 14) (status 10))
 (segment (start 77.0382 81.1574) (end 77.0382 82.2594) (width 0.3) (layer F.Cu) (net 12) (status 20))
 (segment (start 87.7316 77.8158) (end 86.8582 78.6892) (width 0.3) (layer F.Cu) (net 12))
 (segment (start 87.7316 77.1658) (end 87.7316 77.8158) (width 0.3) (layer F.Cu) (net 12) (status 10))
 (segment (start 79.5064 78.6892) (end 77.0382 81.1574) (width 0.3) (layer F.Cu) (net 12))
 (segment (start 86.8582 78.6892) (end 79.5064 78.6892) (width 0.3) (layer F.Cu) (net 12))
 (segment (start 94.3898 82.6798) (end 95.3694 82.6798) (width 0.375) (layer F.Cu) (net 6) (status 20))
 (segment (start 92.6846 80.9746) (end 94.3898 82.6798) (width 0.375) (layer F.Cu) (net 6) (status 10))
 (segment (start 93.1678 78.9782) (end 93.1678 76.8096) (width 0.3) (layer F.Cu) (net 2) (status 20))
 (segment (start 95.3694 81.1798) (end 93.1678 78.9782) (width 0.3) (layer F.Cu) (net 2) (status 10))
 (segment (start 78.3082 88.413) (end 78.3082 87.438) (width 0.3) (layer F.Cu) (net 1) (status 20))
 (segment (start 78.80241 88.90721) (end 78.3082 88.413) (width 0.3) (layer F.Cu) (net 1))
 (segment (start 95.31899 88.90721) (end 78.80241 88.90721) (width 0.3) (layer F.Cu) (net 1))
 (segment (start 95.6564 88.5698) (end 95.31899 88.90721) (width 0.3) (layer F.Cu) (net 1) (status 10))
 (segment (start 95.6564 87.376) (end 95.6564 88.5698) (width 0.3) (layer F.Cu) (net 1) (status 30)))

